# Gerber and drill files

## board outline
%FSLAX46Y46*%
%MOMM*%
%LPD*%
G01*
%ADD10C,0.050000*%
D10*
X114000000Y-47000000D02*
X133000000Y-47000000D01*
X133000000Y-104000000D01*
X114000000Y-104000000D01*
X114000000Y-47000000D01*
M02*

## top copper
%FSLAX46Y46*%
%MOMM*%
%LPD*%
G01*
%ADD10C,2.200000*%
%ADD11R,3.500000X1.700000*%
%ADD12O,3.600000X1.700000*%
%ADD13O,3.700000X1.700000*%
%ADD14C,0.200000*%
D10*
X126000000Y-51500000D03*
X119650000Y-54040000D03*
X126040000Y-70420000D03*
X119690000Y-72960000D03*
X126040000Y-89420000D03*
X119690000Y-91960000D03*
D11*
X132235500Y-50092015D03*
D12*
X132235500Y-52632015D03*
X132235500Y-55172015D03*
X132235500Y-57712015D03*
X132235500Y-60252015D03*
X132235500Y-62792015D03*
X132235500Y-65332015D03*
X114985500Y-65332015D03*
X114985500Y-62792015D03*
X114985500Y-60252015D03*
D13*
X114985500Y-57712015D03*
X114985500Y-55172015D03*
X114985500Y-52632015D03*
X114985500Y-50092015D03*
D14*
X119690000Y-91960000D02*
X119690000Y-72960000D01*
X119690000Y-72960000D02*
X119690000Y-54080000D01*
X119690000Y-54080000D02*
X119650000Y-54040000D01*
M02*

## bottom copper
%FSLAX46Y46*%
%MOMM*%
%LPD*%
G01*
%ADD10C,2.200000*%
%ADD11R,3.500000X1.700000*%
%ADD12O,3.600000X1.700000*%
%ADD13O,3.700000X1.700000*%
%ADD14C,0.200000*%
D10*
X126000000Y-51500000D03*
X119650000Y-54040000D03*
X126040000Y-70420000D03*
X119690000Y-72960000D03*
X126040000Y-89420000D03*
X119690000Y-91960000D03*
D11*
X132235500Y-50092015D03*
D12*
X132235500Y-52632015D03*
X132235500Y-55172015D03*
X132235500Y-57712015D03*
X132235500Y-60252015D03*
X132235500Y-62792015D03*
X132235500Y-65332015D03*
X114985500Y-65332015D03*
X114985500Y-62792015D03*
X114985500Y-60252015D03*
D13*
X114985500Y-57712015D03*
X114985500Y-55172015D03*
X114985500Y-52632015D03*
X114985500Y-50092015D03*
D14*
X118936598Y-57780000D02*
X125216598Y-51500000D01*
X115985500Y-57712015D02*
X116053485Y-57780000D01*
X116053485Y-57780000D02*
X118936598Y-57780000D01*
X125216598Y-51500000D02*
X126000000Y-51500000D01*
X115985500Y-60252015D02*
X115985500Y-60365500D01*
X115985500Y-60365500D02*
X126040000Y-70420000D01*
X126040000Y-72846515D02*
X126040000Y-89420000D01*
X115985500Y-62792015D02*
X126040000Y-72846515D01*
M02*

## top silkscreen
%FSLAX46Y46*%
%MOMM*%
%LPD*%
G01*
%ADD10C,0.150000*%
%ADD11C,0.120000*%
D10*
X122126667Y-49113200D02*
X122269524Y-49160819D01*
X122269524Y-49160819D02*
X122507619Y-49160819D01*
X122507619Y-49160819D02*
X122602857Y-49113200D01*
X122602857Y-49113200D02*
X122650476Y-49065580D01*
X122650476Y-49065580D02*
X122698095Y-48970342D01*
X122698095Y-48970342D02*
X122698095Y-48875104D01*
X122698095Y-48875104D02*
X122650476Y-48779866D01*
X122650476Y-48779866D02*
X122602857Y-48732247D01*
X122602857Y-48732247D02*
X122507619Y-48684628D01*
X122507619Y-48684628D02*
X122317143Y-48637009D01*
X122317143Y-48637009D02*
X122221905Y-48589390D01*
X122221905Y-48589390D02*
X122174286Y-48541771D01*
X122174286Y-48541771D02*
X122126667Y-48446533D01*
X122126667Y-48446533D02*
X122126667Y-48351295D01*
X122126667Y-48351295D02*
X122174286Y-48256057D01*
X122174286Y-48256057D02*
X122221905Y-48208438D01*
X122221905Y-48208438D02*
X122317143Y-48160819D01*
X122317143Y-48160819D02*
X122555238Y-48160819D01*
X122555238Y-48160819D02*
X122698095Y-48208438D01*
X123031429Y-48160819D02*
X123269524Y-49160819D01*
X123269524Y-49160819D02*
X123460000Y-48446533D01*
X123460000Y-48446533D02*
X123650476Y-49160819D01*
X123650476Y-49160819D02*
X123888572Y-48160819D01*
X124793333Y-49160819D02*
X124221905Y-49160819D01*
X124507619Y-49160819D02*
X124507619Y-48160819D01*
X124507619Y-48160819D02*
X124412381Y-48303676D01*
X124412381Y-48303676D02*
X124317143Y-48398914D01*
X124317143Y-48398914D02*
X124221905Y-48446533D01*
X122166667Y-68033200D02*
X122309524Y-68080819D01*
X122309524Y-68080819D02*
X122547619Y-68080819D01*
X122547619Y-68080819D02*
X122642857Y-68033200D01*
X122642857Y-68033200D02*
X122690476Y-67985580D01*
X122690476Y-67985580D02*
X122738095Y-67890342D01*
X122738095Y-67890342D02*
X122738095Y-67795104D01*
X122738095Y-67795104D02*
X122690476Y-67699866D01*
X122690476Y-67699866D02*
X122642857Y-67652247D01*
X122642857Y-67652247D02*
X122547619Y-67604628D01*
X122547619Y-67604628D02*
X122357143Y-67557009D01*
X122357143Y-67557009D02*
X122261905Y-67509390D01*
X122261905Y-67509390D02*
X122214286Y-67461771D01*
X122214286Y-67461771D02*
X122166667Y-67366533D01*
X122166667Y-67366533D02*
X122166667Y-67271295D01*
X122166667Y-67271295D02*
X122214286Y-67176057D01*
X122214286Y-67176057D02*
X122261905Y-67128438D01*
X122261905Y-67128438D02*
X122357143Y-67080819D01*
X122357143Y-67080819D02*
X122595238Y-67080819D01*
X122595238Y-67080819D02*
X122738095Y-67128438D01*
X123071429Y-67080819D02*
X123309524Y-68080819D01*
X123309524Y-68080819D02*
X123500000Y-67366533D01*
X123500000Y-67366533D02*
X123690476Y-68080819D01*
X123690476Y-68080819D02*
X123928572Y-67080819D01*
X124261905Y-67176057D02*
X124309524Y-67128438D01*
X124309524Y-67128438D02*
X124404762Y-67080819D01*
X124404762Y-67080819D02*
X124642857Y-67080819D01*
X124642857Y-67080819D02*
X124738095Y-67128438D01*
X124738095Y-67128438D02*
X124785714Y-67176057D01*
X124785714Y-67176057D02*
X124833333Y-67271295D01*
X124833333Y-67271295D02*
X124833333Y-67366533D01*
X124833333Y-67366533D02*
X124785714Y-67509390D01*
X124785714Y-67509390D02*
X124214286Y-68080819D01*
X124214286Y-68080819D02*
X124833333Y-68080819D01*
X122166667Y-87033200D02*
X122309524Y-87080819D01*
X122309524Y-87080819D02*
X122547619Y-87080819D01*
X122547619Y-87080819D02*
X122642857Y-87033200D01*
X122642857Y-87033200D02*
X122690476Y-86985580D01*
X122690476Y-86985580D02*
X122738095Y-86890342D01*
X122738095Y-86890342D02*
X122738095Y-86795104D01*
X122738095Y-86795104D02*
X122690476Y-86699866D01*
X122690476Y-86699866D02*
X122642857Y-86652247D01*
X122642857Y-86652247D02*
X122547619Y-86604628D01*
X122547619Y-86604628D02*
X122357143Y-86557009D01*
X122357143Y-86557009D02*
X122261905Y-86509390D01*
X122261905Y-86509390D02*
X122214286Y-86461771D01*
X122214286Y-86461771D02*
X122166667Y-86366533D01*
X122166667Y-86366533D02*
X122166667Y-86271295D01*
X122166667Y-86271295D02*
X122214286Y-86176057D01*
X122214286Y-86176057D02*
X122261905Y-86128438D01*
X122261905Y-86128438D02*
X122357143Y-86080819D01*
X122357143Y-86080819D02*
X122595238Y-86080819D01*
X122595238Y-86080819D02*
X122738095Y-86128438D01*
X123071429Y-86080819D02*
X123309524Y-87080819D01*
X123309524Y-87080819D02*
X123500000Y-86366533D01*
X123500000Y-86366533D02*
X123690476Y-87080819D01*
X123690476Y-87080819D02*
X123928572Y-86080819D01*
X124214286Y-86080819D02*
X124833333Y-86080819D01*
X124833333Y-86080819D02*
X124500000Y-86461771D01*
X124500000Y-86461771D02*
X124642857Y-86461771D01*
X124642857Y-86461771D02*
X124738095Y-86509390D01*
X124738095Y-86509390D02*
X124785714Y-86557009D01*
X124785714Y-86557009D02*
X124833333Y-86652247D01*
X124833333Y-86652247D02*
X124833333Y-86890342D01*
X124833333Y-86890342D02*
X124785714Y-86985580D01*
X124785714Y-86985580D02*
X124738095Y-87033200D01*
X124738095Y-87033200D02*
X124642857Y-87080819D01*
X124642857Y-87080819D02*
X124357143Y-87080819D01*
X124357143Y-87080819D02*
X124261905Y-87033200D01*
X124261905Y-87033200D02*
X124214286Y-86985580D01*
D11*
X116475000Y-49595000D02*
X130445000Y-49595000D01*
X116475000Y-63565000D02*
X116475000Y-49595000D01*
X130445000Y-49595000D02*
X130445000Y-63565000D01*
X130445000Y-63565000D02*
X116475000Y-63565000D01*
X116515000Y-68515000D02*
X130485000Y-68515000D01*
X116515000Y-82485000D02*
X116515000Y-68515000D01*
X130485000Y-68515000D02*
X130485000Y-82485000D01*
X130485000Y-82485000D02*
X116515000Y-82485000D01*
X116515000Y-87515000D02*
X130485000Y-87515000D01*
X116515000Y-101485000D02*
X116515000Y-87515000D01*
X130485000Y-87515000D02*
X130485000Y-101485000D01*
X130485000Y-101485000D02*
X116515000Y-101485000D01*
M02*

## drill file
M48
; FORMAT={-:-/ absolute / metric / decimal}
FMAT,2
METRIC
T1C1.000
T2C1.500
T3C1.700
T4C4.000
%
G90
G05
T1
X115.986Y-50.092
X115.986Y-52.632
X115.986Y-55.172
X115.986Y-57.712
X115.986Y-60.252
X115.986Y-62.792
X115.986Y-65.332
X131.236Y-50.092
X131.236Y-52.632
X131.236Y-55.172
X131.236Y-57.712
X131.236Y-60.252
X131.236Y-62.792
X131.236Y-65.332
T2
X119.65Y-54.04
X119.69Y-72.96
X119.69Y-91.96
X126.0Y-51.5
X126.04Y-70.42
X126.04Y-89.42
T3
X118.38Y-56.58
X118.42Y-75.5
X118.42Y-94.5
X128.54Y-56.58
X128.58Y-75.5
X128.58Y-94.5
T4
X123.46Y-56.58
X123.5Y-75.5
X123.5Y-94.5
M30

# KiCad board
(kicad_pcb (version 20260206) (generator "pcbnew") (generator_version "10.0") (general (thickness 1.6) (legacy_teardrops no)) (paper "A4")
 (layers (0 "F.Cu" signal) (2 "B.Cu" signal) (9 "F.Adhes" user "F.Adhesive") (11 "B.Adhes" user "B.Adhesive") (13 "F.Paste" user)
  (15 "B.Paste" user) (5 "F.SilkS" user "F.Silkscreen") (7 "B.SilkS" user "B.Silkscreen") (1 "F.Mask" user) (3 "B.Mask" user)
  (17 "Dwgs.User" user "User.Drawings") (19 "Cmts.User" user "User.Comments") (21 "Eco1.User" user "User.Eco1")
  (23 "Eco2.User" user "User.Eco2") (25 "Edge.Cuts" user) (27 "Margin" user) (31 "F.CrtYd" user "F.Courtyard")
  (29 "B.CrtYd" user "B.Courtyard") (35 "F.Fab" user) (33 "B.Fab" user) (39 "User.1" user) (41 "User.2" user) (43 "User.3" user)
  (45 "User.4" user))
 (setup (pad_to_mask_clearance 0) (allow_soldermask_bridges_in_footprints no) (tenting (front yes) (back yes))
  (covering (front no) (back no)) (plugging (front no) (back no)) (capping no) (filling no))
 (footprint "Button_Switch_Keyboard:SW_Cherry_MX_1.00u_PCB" (layer "F.Cu") (at 126 51.5)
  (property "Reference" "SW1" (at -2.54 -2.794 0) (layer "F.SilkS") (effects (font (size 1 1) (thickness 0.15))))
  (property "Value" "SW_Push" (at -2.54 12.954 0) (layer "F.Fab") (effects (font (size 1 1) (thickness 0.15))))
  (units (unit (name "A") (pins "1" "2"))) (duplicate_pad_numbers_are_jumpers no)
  (fp_line (start -9.525 -1.905) (end 4.445 -1.905) (stroke (width 0.12) (type solid)) (layer "F.SilkS"))
  (fp_line (start -9.525 12.065) (end -9.525 -1.905) (stroke (width 0.12) (type solid)) (layer "F.SilkS"))
  (fp_line (start 4.445 -1.905) (end 4.445 12.065) (stroke (width 0.12) (type solid)) (layer "F.SilkS"))
  (fp_line (start 4.445 12.065) (end -9.525 12.065) (stroke (width 0.12) (type solid)) (layer "F.SilkS"))
  (pad "" np_thru_hole circle (at -7.62 5.08) (size 1.7 1.7) (drill 1.7) (layers "*.Cu" "*.Mask"))
  (pad "" np_thru_hole circle (at -2.54 5.08) (size 4 4) (drill 4) (layers "*.Cu" "*.Mask"))
  (pad "" np_thru_hole circle (at 2.54 5.08) (size 1.7 1.7) (drill 1.7) (layers "*.Cu" "*.Mask"))
  (pad "1" thru_hole circle (at 0 0) (size 2.2 2.2) (drill 1.5) (layers "*.Cu" "*.Mask") (remove_unused_layers no)
   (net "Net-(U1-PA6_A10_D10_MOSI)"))
  (pad "2" thru_hole circle (at -6.35 2.54) (size 2.2 2.2) (drill 1.5) (layers "*.Cu" "*.Mask") (remove_unused_layers no) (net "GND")))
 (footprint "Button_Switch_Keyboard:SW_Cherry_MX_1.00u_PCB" (layer "F.Cu") (at 126.04 70.42)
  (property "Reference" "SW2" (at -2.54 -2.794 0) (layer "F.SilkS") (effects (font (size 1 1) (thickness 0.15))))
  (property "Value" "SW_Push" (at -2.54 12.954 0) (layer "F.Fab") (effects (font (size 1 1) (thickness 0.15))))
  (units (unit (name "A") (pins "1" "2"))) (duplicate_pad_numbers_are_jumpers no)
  (fp_line (start -9.525 -1.905) (end 4.445 -1.905) (stroke (width 0.12) (type solid)) (layer "F.SilkS"))
  (fp_line (start -9.525 12.065) (end -9.525 -1.905) (stroke (width 0.12) (type solid)) (layer "F.SilkS"))
  (fp_line (start 4.445 -1.905) (end 4.445 12.065) (stroke (width 0.12) (type solid)) (layer "F.SilkS"))
  (fp_line (start 4.445 12.065) (end -9.525 12.065) (stroke (width 0.12) (type solid)) (layer "F.SilkS"))
  (pad "" np_thru_hole circle (at -7.62 5.08) (size 1.7 1.7) (drill 1.7) (layers "*.Cu" "*.Mask"))
  (pad "" np_thru_hole circle (at -2.54 5.08) (size 4 4) (drill 4) (layers "*.Cu" "*.Mask"))
  (pad "" np_thru_hole circle (at 2.54 5.08) (size 1.7 1.7) (drill 1.7) (layers "*.Cu" "*.Mask"))
  (pad "1" thru_hole circle (at 0 0) (size 2.2 2.2) (drill 1.5) (layers "*.Cu" "*.Mask") (remove_unused_layers no)
   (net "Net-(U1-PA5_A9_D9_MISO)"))
  (pad "2" thru_hole circle (at -6.35 2.54) (size 2.2 2.2) (drill 1.5) (layers "*.Cu" "*.Mask") (remove_unused_layers no) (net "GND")))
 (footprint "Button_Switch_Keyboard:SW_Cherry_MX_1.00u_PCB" (layer "F.Cu") (at 126.04 89.42)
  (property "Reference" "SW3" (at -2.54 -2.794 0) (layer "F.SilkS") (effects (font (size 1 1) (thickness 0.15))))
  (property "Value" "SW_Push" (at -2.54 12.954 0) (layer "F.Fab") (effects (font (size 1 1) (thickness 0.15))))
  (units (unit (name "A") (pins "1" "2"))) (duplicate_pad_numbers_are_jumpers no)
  (fp_line (start -9.525 -1.905) (end 4.445 -1.905) (stroke (width 0.12) (type solid)) (layer "F.SilkS"))
  (fp_line (start -9.525 12.065) (end -9.525 -1.905) (stroke (width 0.12) (type solid)) (layer "F.SilkS"))
  (fp_line (start 4.445 -1.905) (end 4.445 12.065) (stroke (width 0.12) (type solid)) (layer "F.SilkS"))
  (fp_line (start 4.445 12.065) (end -9.525 12.065) (stroke (width 0.12) (type solid)) (layer "F.SilkS"))
  (pad "" np_thru_hole circle (at -7.62 5.08) (size 1.7 1.7) (drill 1.7) (layers "*.Cu" "*.Mask"))
  (pad "" np_thru_hole circle (at -2.54 5.08) (size 4 4) (drill 4) (layers "*.Cu" "*.Mask"))
  (pad "" np_thru_hole circle (at 2.54 5.08) (size 1.7 1.7) (drill 1.7) (layers "*.Cu" "*.Mask"))
  (pad "1" thru_hole circle (at 0 0) (size 2.2 2.2) (drill 1.5) (layers "*.Cu" "*.Mask") (remove_unused_layers no)
   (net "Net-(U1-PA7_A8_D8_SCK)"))
  (pad "2" thru_hole circle (at -6.35 2.54) (size 2.2 2.2) (drill 1.5) (layers "*.Cu" "*.Mask") (remove_unused_layers no) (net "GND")))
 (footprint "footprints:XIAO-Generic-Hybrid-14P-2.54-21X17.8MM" (layer "B.Cu") (at 123.6105 57.712015 180)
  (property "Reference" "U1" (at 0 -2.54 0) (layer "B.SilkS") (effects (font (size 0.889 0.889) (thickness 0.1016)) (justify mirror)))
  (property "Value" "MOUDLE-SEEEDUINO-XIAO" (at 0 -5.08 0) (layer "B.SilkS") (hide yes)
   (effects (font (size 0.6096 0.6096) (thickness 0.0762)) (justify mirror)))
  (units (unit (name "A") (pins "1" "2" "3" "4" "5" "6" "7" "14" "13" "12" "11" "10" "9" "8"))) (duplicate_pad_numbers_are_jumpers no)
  (pad "1" thru_hole rect (at -7.625 7.62 180) (size 3.5 1.7) (drill 1 (offset -1 0)) (layers "*.Cu" "*.Mask") (remove_unused_layers no)
   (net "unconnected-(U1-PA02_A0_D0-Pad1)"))
  (pad "2" thru_hole oval (at -7.625 5.08 180) (size 3.6 1.7) (drill 1 (offset -1 0)) (layers "*.Cu" "*.Mask") (remove_unused_layers no)
   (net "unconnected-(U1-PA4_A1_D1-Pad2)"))
  (pad "3" thru_hole oval (at -7.625 2.54 180) (size 3.6 1.7) (drill 1 (offset -1 0)) (layers "*.Cu" "*.Mask") (remove_unused_layers no)
   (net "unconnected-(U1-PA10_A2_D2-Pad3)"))
  (pad "4" thru_hole oval (at -7.625 0 180) (size 3.6 1.7) (drill 1 (offset -1 0)) (layers "*.Cu" "*.Mask") (remove_unused_layers no)
   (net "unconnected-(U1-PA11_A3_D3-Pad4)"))
  (pad "5" thru_hole oval (at -7.625 -2.54 180) (size 3.6 1.7) (drill 1 (offset -1 0)) (layers "*.Cu" "*.Mask") (remove_unused_layers no)
   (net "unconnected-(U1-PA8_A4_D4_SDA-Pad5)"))
  (pad "6" thru_hole oval (at -7.625 -5.08) (size 3.6 1.7) (drill 1 (offset 1 0)) (layers "*.Cu" "*.Mask") (remove_unused_layers no)
   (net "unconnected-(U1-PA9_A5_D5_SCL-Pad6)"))
  (pad "7" thru_hole oval (at -7.625 -7.62 180) (size 3.6 1.7) (drill 1 (offset -1 0)) (layers "*.Cu" "*.Mask") (remove_unused_layers no)
   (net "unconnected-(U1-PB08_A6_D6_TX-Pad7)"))
  (pad "8" thru_hole oval (at 7.625 -7.62 180) (size 3.6 1.7) (drill 1 (offset 1 0)) (layers "*.Cu" "*.Mask") (remove_unused_layers no)
   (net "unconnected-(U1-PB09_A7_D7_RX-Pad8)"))
  (pad "9" thru_hole oval (at 7.625 -5.08 180) (size 3.6 1.7) (drill 1 (offset 1 0)) (layers "*.Cu" "*.Mask") (remove_unused_layers no)
   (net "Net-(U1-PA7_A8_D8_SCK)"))
  (pad "10" thru_hole oval (at 7.625 -2.54 180) (size 3.6 1.7) (drill 1 (offset 1 0)) (layers "*.Cu" "*.Mask") (remove_unused_layers no)
   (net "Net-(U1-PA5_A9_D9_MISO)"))
  (pad "11" thru_hole oval (at 7.625 0 180) (size 3.7 1.7) (drill 1 (offset 1 0)) (layers "*.Cu" "*.Mask") (remove_unused_layers no)
   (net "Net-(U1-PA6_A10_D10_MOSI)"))
  (pad "12" thru_hole oval (at 7.625 2.54 180) (size 3.7 1.7) (drill 1 (offset 1 0)) (layers "*.Cu" "*.Mask") (remove_unused_layers no)
   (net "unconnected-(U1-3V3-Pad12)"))
  (pad "13" thru_hole oval (at 7.625 5.08 180) (size 3.7 1.7) (drill 1 (offset 1 0)) (layers "*.Cu" "*.Mask") (remove_unused_layers no)
   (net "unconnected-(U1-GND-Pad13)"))
  (pad "14" thru_hole oval (at 7.625 7.62 180) (size 3.7 1.7) (drill 1 (offset 1 0)) (layers "*.Cu" "*.Mask") (remove_unused_layers no)
   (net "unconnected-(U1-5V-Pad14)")))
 (gr_rect (start 114 47) (end 133 104) (stroke (width 0.05) (type default)) (fill no) (layer "Edge.Cuts"))
 (segment (start 119.69 91.96) (end 119.69 72.96) (width 0.2) (layer "F.Cu") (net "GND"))
 (segment (start 119.69 72.96) (end 119.69 54.08) (width 0.2) (layer "F.Cu") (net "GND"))
 (segment (start 119.69 54.08) (end 119.65 54.04) (width 0.2) (layer "F.Cu") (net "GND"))
 (segment (start 118.936598 57.78) (end 125.216598 51.5) (width 0.2) (layer "B.Cu") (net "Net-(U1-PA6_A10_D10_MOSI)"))
 (segment (start 115.9855 57.712015) (end 116.053485 57.78) (width 0.2) (layer "B.Cu") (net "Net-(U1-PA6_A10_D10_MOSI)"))
 (segment (start 116.053485 57.78) (end 118.936598 57.78) (width 0.2) (layer "B.Cu") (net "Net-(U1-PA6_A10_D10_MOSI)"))
 (segment (start 125.216598 51.5) (end 126 51.5) (width 0.2) (layer "B.Cu") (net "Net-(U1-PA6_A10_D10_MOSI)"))
 (segment (start 115.9855 60.252015) (end 115.9855 60.3655) (width 0.2) (layer "B.Cu") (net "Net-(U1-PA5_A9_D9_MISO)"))
 (segment (start 115.9855 60.3655) (end 126.04 70.42) (width 0.2) (layer "B.Cu") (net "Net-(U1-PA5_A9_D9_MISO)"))
 (segment (start 126.04 72.846515) (end 126.04 89.42) (width 0.2) (layer "B.Cu") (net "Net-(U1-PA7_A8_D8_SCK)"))
 (segment (start 115.9855 62.792015) (end 126.04 72.846515) (width 0.2) (layer "B.Cu") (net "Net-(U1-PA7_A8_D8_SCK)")))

